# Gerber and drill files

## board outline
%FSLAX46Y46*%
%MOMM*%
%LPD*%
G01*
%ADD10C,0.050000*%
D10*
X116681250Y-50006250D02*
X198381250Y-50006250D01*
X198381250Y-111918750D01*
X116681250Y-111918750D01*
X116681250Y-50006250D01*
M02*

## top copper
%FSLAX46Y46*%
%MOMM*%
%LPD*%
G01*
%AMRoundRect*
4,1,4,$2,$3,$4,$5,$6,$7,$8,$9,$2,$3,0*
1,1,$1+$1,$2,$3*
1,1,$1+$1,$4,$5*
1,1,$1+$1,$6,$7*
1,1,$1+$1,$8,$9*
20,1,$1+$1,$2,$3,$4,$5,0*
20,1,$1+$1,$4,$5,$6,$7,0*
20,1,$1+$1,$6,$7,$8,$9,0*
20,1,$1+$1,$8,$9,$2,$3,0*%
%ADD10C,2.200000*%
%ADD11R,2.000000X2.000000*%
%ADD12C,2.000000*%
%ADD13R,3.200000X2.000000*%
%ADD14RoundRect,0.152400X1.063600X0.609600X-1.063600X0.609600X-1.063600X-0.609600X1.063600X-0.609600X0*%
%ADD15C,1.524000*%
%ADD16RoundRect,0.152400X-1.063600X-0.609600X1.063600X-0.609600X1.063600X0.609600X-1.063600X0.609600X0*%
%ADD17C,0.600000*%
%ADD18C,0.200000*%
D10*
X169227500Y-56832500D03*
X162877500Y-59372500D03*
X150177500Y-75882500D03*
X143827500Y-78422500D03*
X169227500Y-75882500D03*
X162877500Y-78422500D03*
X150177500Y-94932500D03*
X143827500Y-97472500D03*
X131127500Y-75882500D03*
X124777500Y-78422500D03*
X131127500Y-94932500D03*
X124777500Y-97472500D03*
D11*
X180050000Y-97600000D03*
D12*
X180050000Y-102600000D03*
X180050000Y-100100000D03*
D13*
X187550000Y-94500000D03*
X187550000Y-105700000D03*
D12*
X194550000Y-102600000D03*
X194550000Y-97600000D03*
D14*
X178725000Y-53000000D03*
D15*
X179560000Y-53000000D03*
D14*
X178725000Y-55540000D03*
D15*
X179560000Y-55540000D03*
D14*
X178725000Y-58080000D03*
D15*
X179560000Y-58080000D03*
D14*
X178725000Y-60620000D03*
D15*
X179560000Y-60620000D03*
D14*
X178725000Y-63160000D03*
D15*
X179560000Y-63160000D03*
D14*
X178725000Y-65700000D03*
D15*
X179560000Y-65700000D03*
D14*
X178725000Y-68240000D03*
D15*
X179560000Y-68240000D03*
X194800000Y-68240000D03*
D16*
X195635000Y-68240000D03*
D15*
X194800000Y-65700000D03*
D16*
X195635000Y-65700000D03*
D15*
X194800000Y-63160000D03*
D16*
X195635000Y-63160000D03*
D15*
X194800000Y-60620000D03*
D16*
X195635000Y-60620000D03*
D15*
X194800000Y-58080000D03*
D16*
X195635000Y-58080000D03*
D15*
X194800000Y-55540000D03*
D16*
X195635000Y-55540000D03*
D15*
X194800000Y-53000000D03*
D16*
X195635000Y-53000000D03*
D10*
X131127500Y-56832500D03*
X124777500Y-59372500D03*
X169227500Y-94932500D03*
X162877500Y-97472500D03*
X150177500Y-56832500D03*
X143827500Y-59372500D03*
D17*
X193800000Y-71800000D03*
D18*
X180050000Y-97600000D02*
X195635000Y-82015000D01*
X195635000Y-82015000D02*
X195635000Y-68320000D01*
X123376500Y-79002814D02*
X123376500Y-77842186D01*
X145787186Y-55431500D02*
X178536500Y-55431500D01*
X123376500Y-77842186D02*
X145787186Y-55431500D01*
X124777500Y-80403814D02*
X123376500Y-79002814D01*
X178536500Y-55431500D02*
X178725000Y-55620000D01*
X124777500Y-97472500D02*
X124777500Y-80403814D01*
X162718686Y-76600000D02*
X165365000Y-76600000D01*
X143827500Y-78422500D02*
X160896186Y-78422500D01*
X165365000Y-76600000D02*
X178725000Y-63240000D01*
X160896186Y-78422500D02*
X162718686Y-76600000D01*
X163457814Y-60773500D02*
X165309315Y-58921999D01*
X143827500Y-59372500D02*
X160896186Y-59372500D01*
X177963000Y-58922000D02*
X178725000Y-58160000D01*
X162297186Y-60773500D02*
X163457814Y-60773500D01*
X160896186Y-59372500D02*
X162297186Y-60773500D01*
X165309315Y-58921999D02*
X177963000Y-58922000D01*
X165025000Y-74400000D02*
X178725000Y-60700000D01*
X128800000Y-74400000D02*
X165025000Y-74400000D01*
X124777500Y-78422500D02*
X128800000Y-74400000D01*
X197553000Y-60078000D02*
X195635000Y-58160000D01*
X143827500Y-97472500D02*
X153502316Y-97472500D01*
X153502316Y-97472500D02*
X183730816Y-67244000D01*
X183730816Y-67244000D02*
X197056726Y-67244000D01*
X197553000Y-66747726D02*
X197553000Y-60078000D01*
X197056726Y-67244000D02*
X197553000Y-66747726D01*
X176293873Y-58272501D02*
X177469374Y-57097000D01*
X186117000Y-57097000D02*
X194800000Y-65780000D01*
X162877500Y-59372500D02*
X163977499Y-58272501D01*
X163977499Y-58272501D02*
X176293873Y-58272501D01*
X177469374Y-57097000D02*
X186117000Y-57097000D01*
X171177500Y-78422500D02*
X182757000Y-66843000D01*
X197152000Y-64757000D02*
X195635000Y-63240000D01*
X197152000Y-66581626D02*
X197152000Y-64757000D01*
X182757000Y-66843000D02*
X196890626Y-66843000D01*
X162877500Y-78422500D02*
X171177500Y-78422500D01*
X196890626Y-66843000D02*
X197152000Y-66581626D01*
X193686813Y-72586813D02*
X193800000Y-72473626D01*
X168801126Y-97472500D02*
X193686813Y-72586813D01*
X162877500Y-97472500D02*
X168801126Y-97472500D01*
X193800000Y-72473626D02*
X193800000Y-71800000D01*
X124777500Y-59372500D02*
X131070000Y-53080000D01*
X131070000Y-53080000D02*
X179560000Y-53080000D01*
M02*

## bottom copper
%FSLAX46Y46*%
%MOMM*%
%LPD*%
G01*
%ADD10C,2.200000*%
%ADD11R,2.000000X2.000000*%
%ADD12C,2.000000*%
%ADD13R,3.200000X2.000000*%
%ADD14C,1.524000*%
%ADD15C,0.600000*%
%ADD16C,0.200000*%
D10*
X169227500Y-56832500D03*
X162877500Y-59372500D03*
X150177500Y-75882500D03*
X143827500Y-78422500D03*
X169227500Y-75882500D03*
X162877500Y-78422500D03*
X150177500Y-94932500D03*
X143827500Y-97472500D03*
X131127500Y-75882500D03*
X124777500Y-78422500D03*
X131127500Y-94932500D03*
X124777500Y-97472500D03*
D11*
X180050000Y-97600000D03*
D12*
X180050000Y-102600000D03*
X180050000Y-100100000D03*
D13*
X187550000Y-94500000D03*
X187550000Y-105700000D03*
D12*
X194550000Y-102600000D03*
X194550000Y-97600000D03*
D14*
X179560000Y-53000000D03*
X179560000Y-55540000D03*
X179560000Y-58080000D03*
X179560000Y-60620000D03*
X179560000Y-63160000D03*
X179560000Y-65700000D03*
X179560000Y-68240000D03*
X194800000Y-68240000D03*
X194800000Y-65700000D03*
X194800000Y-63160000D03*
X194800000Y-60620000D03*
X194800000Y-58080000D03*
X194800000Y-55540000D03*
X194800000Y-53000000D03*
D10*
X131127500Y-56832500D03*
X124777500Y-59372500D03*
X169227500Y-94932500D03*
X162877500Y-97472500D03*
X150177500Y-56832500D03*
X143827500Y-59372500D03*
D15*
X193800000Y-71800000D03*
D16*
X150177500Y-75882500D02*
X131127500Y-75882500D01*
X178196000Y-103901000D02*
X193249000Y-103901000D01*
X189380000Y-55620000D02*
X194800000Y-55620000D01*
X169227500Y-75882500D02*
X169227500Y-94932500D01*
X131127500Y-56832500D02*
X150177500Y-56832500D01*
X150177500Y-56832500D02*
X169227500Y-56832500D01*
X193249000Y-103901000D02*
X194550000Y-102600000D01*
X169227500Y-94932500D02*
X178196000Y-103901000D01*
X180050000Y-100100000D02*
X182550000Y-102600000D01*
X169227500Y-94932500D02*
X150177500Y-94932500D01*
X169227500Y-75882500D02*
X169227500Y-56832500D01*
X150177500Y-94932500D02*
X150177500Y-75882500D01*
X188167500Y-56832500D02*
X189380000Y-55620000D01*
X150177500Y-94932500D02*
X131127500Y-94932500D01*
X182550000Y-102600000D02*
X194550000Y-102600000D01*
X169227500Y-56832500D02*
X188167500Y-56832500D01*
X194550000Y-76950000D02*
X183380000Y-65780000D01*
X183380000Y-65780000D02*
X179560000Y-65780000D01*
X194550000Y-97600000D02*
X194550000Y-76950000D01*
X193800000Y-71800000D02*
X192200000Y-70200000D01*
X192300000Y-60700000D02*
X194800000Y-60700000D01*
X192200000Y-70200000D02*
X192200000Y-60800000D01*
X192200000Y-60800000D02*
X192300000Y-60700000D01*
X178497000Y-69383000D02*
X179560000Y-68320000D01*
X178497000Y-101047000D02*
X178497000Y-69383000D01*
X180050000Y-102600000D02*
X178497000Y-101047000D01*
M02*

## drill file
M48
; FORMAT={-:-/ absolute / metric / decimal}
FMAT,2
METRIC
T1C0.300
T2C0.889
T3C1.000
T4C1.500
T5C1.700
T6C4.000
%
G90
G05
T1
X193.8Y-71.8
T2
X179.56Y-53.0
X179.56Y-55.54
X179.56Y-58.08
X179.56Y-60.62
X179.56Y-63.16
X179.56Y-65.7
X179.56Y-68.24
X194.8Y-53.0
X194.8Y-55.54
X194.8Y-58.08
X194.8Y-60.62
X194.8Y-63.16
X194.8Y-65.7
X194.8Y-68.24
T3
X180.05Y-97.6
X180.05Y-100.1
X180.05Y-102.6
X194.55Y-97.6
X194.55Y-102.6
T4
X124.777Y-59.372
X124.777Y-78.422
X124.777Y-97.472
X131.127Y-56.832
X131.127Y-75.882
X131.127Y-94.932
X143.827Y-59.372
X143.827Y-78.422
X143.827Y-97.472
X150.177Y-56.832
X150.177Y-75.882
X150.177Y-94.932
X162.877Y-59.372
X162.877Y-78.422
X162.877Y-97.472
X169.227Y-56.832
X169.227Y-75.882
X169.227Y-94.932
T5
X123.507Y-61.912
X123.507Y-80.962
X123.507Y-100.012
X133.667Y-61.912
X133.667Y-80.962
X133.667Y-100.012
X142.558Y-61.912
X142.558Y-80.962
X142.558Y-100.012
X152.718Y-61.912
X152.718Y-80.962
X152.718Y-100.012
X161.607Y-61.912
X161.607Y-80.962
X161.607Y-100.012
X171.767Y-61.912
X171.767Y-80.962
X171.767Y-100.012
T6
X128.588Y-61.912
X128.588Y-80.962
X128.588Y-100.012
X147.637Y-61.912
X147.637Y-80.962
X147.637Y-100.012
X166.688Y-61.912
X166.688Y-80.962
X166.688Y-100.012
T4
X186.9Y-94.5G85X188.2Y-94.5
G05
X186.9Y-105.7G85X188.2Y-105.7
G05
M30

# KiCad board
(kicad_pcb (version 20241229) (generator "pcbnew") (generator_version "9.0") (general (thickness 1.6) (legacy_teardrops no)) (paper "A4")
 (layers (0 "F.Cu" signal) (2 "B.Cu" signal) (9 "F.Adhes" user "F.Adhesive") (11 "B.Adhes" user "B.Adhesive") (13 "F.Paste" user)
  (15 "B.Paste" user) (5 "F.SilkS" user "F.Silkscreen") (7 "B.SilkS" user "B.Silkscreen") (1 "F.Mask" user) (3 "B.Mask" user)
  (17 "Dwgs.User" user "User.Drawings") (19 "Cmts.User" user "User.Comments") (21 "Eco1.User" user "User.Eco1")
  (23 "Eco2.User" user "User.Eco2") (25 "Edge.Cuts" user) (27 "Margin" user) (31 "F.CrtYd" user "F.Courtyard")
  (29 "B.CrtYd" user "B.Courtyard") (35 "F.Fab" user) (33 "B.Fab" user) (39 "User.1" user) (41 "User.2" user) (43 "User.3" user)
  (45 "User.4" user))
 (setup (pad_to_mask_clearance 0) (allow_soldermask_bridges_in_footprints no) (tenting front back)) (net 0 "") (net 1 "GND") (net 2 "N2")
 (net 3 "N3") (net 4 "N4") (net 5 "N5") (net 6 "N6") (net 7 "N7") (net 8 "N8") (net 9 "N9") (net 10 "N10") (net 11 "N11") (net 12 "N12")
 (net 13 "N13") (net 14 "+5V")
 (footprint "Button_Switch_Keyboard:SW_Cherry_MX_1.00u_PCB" (layer "F.Cu") (at 169.2275 56.8325)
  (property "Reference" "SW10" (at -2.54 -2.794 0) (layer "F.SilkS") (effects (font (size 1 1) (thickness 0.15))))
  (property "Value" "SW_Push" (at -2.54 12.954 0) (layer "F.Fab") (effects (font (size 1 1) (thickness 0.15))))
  (pad "" np_thru_hole circle (at -7.62 5.08) (size 1.7 1.7) (drill 1.7) (layers "*.Cu" "*.Mask"))
  (pad "" np_thru_hole circle (at -2.54 5.08) (size 4 4) (drill 4) (layers "*.Cu" "*.Mask"))
  (pad "" np_thru_hole circle (at 2.54 5.08) (size 1.7 1.7) (drill 1.7) (layers "*.Cu" "*.Mask"))
  (pad "1" thru_hole circle (at 0 0) (size 2.2 2.2) (drill 1.5) (layers "*.Cu" "*.Mask") (remove_unused_layers no) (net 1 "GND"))
  (pad "2" thru_hole circle (at -6.35 2.54) (size 2.2 2.2) (drill 1.5) (layers "*.Cu" "*.Mask") (remove_unused_layers no) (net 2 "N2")))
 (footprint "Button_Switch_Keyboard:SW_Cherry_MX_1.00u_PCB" (layer "F.Cu") (at 150.1775 75.8825)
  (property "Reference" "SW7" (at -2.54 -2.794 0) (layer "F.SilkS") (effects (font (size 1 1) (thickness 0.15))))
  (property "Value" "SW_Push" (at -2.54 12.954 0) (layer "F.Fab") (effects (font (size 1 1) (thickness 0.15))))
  (pad "" np_thru_hole circle (at -7.62 5.08) (size 1.7 1.7) (drill 1.7) (layers "*.Cu" "*.Mask"))
  (pad "" np_thru_hole circle (at -2.54 5.08) (size 4 4) (drill 4) (layers "*.Cu" "*.Mask"))
  (pad "" np_thru_hole circle (at 2.54 5.08) (size 1.7 1.7) (drill 1.7) (layers "*.Cu" "*.Mask"))
  (pad "1" thru_hole circle (at 0 0) (size 2.2 2.2) (drill 1.5) (layers "*.Cu" "*.Mask") (remove_unused_layers no) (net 1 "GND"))
  (pad "2" thru_hole circle (at -6.35 2.54) (size 2.2 2.2) (drill 1.5) (layers "*.Cu" "*.Mask") (remove_unused_layers no) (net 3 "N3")))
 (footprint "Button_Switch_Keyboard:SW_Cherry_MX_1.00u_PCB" (layer "F.Cu") (at 169.2275 75.8825)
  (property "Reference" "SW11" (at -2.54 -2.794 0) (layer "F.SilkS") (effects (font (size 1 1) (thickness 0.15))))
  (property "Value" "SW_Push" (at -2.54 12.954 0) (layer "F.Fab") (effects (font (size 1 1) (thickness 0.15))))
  (pad "" np_thru_hole circle (at -7.62 5.08) (size 1.7 1.7) (drill 1.7) (layers "*.Cu" "*.Mask"))
  (pad "" np_thru_hole circle (at -2.54 5.08) (size 4 4) (drill 4) (layers "*.Cu" "*.Mask"))
  (pad "" np_thru_hole circle (at 2.54 5.08) (size 1.7 1.7) (drill 1.7) (layers "*.Cu" "*.Mask"))
  (pad "1" thru_hole circle (at 0 0) (size 2.2 2.2) (drill 1.5) (layers "*.Cu" "*.Mask") (remove_unused_layers no) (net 1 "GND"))
  (pad "2" thru_hole circle (at -6.35 2.54) (size 2.2 2.2) (drill 1.5) (layers "*.Cu" "*.Mask") (remove_unused_layers no) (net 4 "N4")))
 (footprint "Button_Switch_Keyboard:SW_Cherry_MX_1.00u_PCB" (layer "F.Cu") (at 150.1775 94.9325)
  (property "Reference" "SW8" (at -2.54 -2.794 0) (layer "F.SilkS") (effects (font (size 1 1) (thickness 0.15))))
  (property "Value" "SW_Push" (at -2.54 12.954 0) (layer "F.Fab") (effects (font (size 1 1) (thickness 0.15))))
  (pad "" np_thru_hole circle (at -7.62 5.08) (size 1.7 1.7) (drill 1.7) (layers "*.Cu" "*.Mask"))
  (pad "" np_thru_hole circle (at -2.54 5.08) (size 4 4) (drill 4) (layers "*.Cu" "*.Mask"))
  (pad "" np_thru_hole circle (at 2.54 5.08) (size 1.7 1.7) (drill 1.7) (layers "*.Cu" "*.Mask"))
  (pad "1" thru_hole circle (at 0 0) (size 2.2 2.2) (drill 1.5) (layers "*.Cu" "*.Mask") (remove_unused_layers no) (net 1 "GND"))
  (pad "2" thru_hole circle (at -6.35 2.54) (size 2.2 2.2) (drill 1.5) (layers "*.Cu" "*.Mask") (remove_unused_layers no) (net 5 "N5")))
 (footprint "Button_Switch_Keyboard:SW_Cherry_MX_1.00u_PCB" (layer "F.Cu") (at 131.1275 75.8825)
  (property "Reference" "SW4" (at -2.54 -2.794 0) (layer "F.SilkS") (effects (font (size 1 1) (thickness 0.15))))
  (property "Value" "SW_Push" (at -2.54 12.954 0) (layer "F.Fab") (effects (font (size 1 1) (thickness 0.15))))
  (pad "" np_thru_hole circle (at -7.62 5.08) (size 1.7 1.7) (drill 1.7) (layers "*.Cu" "*.Mask"))
  (pad "" np_thru_hole circle (at -2.54 5.08) (size 4 4) (drill 4) (layers "*.Cu" "*.Mask"))
  (pad "" np_thru_hole circle (at 2.54 5.08) (size 1.7 1.7) (drill 1.7) (layers "*.Cu" "*.Mask"))
  (pad "1" thru_hole circle (at 0 0) (size 2.2 2.2) (drill 1.5) (layers "*.Cu" "*.Mask") (remove_unused_layers no) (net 1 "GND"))
  (pad "2" thru_hole circle (at -6.35 2.54) (size 2.2 2.2) (drill 1.5) (layers "*.Cu" "*.Mask") (remove_unused_layers no) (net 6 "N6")))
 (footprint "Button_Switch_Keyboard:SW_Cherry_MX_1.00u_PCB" (layer "F.Cu") (at 131.1275 94.9325)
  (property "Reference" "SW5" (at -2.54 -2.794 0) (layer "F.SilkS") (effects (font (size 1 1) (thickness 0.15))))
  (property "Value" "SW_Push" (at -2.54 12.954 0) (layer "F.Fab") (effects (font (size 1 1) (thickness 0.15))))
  (pad "" np_thru_hole circle (at -7.62 5.08) (size 1.7 1.7) (drill 1.7) (layers "*.Cu" "*.Mask"))
  (pad "" np_thru_hole circle (at -2.54 5.08) (size 4 4) (drill 4) (layers "*.Cu" "*.Mask"))
  (pad "" np_thru_hole circle (at 2.54 5.08) (size 1.7 1.7) (drill 1.7) (layers "*.Cu" "*.Mask"))
  (pad "1" thru_hole circle (at 0 0) (size 2.2 2.2) (drill 1.5) (layers "*.Cu" "*.Mask") (remove_unused_layers no) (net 1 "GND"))
  (pad "2" thru_hole circle (at -6.35 2.54) (size 2.2 2.2) (drill 1.5) (layers "*.Cu" "*.Mask") (remove_unused_layers no) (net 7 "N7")))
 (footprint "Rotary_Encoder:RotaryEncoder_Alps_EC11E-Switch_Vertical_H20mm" (layer "F.Cu") (at 180.05 97.6)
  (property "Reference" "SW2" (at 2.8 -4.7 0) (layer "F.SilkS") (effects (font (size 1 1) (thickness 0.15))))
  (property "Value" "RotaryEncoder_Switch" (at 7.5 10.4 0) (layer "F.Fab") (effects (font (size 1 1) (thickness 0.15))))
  (pad "A" thru_hole rect (at 0 0) (size 2 2) (drill 1) (layers "*.Cu" "*.Mask") (remove_unused_layers no) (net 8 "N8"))
  (pad "B" thru_hole circle (at 0 5) (size 2 2) (drill 1) (layers "*.Cu" "*.Mask") (remove_unused_layers no) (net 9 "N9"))
  (pad "C" thru_hole circle (at 0 2.5) (size 2 2) (drill 1) (layers "*.Cu" "*.Mask") (remove_unused_layers no) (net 1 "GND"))
  (pad "MP" thru_hole rect (at 7.5 -3.1) (size 3.2 2) (drill oval 2.8 1.5) (layers "*.Cu" "*.Mask") (remove_unused_layers no))
  (pad "MP" thru_hole rect (at 7.5 8.1) (size 3.2 2) (drill oval 2.8 1.5) (layers "*.Cu" "*.Mask") (remove_unused_layers no))
  (pad "S1" thru_hole circle (at 14.5 5) (size 2 2) (drill 1) (layers "*.Cu" "*.Mask") (remove_unused_layers no) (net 1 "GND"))
  (pad "S2" thru_hole circle (at 14.5 0) (size 2 2) (drill 1) (layers "*.Cu" "*.Mask") (remove_unused_layers no) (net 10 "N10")))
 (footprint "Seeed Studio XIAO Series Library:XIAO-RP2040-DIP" (layer "F.Cu") (at 187.18 60.62)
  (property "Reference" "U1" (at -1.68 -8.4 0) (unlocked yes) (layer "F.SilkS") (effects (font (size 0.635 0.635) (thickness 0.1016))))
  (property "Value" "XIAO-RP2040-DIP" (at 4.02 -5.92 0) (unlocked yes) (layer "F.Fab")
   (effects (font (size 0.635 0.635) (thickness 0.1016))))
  (pad "1" smd roundrect (at -8.455 -7.62 180) (size 2.432 1.524) (layers "F.Cu" "F.Mask") (roundrect_rratio 0.1) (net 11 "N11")
   (thermal_bridge_angle 45))
  (pad "1" thru_hole circle (at -7.62 -7.62 180) (size 1.524 1.524) (drill 0.889) (layers "*.Cu" "*.Mask") (remove_unused_layers no)
   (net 11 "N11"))
  (pad "2" smd roundrect (at -8.455 -5.08 180) (size 2.432 1.524) (layers "F.Cu" "F.Mask") (roundrect_rratio 0.1) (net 7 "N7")
   (thermal_bridge_angle 45))
  (pad "2" thru_hole circle (at -7.62 -5.08 180) (size 1.524 1.524) (drill 0.889) (layers "*.Cu" "*.Mask") (remove_unused_layers no)
   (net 7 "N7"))
  (pad "3" smd roundrect (at -8.455 -2.54 180) (size 2.432 1.524) (layers "F.Cu" "F.Mask") (roundrect_rratio 0.1) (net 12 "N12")
   (thermal_bridge_angle 45))
  (pad "3" thru_hole circle (at -7.62 -2.54 180) (size 1.524 1.524) (drill 0.889) (layers "*.Cu" "*.Mask") (remove_unused_layers no)
   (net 12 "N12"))
  (pad "4" smd roundrect (at -8.455 0 180) (size 2.432 1.524) (layers "F.Cu" "F.Mask") (roundrect_rratio 0.1) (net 6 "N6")
   (thermal_bridge_angle 45))
  (pad "4" thru_hole circle (at -7.62 0 180) (size 1.524 1.524) (drill 0.889) (layers "*.Cu" "*.Mask") (remove_unused_layers no)
   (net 6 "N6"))
  (pad "5" smd roundrect (at -8.455 2.54 180) (size 2.432 1.524) (layers "F.Cu" "F.Mask") (roundrect_rratio 0.1) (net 3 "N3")
   (thermal_bridge_angle 45))
  (pad "5" thru_hole circle (at -7.62 2.54 180) (size 1.524 1.524) (drill 0.889) (layers "*.Cu" "*.Mask") (remove_unused_layers no)
   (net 3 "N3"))
  (pad "6" smd roundrect (at -8.455 5.08 180) (size 2.432 1.524) (layers "F.Cu" "F.Mask") (roundrect_rratio 0.1) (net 10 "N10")
   (thermal_bridge_angle 45))
  (pad "6" thru_hole circle (at -7.62 5.08 180) (size 1.524 1.524) (drill 0.889) (layers "*.Cu" "*.Mask") (remove_unused_layers no)
   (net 10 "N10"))
  (pad "7" smd roundrect (at -8.455 7.62 180) (size 2.432 1.524) (layers "F.Cu" "F.Mask") (roundrect_rratio 0.1) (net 9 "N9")
   (thermal_bridge_angle 45))
  (pad "7" thru_hole circle (at -7.62 7.62 180) (size 1.524 1.524) (drill 0.889) (layers "*.Cu" "*.Mask") (remove_unused_layers no)
   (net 9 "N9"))
  (pad "8" thru_hole circle (at 7.62 7.62) (size 1.524 1.524) (drill 0.889) (layers "*.Cu" "*.Mask") (remove_unused_layers no) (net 8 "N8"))
  (pad "8" smd roundrect (at 8.455 7.62) (size 2.432 1.524) (layers "F.Cu" "F.Mask") (roundrect_rratio 0.1) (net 8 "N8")
   (thermal_bridge_angle 45))
  (pad "9" thru_hole circle (at 7.62 5.08) (size 1.524 1.524) (drill 0.889) (layers "*.Cu" "*.Mask") (remove_unused_layers no) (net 2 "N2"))
  (pad "9" smd roundrect (at 8.455 5.08) (size 2.432 1.524) (layers "F.Cu" "F.Mask") (roundrect_rratio 0.1) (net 2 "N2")
   (thermal_bridge_angle 45))
  (pad "10" thru_hole circle (at 7.62 2.54) (size 1.524 1.524) (drill 0.889) (layers "*.Cu" "*.Mask") (remove_unused_layers no) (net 4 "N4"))
  (pad "10" smd roundrect (at 8.455 2.54) (size 2.432 1.524) (layers "F.Cu" "F.Mask") (roundrect_rratio 0.1) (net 4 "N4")
   (thermal_bridge_angle 45))
  (pad "11" thru_hole circle (at 7.62 0) (size 1.524 1.524) (drill 0.889) (layers "*.Cu" "*.Mask") (remove_unused_layers no) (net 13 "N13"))
  (pad "11" smd roundrect (at 8.455 0) (size 2.432 1.524) (layers "F.Cu" "F.Mask") (roundrect_rratio 0.1) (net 13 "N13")
   (thermal_bridge_angle 45))
  (pad "12" thru_hole circle (at 7.62 -2.54) (size 1.524 1.524) (drill 0.889) (layers "*.Cu" "*.Mask") (remove_unused_layers no)
   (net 5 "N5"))
  (pad "12" smd roundrect (at 8.455 -2.54) (size 2.432 1.524) (layers "F.Cu" "F.Mask") (roundrect_rratio 0.1) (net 5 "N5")
   (thermal_bridge_angle 45))
  (pad "13" thru_hole circle (at 7.62 -5.08) (size 1.524 1.524) (drill 0.889) (layers "*.Cu" "*.Mask") (remove_unused_layers no)
   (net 1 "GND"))
  (pad "13" smd roundrect (at 8.455 -5.08) (size 2.432 1.524) (layers "F.Cu" "F.Mask") (roundrect_rratio 0.1) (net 1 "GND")
   (thermal_bridge_angle 45))
  (pad "14" thru_hole circle (at 7.62 -7.62) (size 1.524 1.524) (drill 0.889) (layers "*.Cu" "*.Mask") (remove_unused_layers no)
   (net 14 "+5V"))
  (pad "14" smd roundrect (at 8.455 -7.62) (size 2.432 1.524) (layers "F.Cu" "F.Mask") (roundrect_rratio 0.1) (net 14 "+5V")
   (thermal_bridge_angle 45)))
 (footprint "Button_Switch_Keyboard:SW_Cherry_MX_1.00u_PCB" (layer "F.Cu") (at 131.1275 56.8325)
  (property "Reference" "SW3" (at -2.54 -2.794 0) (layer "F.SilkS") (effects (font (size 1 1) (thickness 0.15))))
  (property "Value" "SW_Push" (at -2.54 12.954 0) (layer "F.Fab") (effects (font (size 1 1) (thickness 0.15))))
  (pad "" np_thru_hole circle (at -7.62 5.08) (size 1.7 1.7) (drill 1.7) (layers "*.Cu" "*.Mask"))
  (pad "" np_thru_hole circle (at -2.54 5.08) (size 4 4) (drill 4) (layers "*.Cu" "*.Mask"))
  (pad "" np_thru_hole circle (at 2.54 5.08) (size 1.7 1.7) (drill 1.7) (layers "*.Cu" "*.Mask"))
  (pad "1" thru_hole circle (at 0 0) (size 2.2 2.2) (drill 1.5) (layers "*.Cu" "*.Mask") (remove_unused_layers no) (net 1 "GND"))
  (pad "2" thru_hole circle (at -6.35 2.54) (size 2.2 2.2) (drill 1.5) (layers "*.Cu" "*.Mask") (remove_unused_layers no) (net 11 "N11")))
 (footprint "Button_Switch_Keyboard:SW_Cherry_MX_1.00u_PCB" (layer "F.Cu") (at 169.2275 94.9325)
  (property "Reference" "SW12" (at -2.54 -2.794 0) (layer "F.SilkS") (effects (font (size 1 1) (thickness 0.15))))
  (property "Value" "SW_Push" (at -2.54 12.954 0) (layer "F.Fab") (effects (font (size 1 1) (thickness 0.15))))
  (pad "" np_thru_hole circle (at -7.62 5.08) (size 1.7 1.7) (drill 1.7) (layers "*.Cu" "*.Mask"))
  (pad "" np_thru_hole circle (at -2.54 5.08) (size 4 4) (drill 4) (layers "*.Cu" "*.Mask"))
  (pad "" np_thru_hole circle (at 2.54 5.08) (size 1.7 1.7) (drill 1.7) (layers "*.Cu" "*.Mask"))
  (pad "1" thru_hole circle (at 0 0) (size 2.2 2.2) (drill 1.5) (layers "*.Cu" "*.Mask") (remove_unused_layers no) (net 1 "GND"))
  (pad "2" thru_hole circle (at -6.35 2.54) (size 2.2 2.2) (drill 1.5) (layers "*.Cu" "*.Mask") (remove_unused_layers no) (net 13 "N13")))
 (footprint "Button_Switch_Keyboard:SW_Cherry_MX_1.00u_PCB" (layer "F.Cu") (at 150.1775 56.8325)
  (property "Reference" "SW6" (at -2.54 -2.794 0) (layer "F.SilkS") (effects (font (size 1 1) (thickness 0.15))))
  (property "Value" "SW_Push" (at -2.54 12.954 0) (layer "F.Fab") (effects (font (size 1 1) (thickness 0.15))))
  (pad "" np_thru_hole circle (at -7.62 5.08) (size 1.7 1.7) (drill 1.7) (layers "*.Cu" "*.Mask"))
  (pad "" np_thru_hole circle (at -2.54 5.08) (size 4 4) (drill 4) (layers "*.Cu" "*.Mask"))
  (pad "" np_thru_hole circle (at 2.54 5.08) (size 1.7 1.7) (drill 1.7) (layers "*.Cu" "*.Mask"))
  (pad "1" thru_hole circle (at 0 0) (size 2.2 2.2) (drill 1.5) (layers "*.Cu" "*.Mask") (remove_unused_layers no) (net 1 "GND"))
  (pad "2" thru_hole circle (at -6.35 2.54) (size 2.2 2.2) (drill 1.5) (layers "*.Cu" "*.Mask") (remove_unused_layers no) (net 12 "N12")))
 (gr_rect (start 116.68125 50.00625) (end 198.38125 111.91875) (stroke (width 0.05) (type default)) (fill no) (layer "Edge.Cuts"))
 (segment (start 150.1775 75.8825) (end 131.1275 75.8825) (width 0.2) (layer "B.Cu") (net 1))
 (segment (start 178.196 103.901) (end 193.249 103.901) (width 0.2) (layer "B.Cu") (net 1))
 (segment (start 189.38 55.62) (end 194.8 55.62) (width 0.2) (layer "B.Cu") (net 1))
 (segment (start 169.2275 75.8825) (end 169.2275 94.9325) (width 0.2) (layer "B.Cu") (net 1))
 (segment (start 131.1275 56.8325) (end 150.1775 56.8325) (width 0.2) (layer "B.Cu") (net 1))
 (segment (start 150.1775 56.8325) (end 169.2275 56.8325) (width 0.2) (layer "B.Cu") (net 1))
 (segment (start 193.249 103.901) (end 194.55 102.6) (width 0.2) (layer "B.Cu") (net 1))
 (segment (start 169.2275 94.9325) (end 178.196 103.901) (width 0.2) (layer "B.Cu") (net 1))
 (segment (start 180.05 100.1) (end 182.55 102.6) (width 0.2) (layer "B.Cu") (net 1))
 (segment (start 169.2275 94.9325) (end 150.1775 94.9325) (width 0.2) (layer "B.Cu") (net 1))
 (segment (start 169.2275 75.8825) (end 169.2275 56.8325) (width 0.2) (layer "B.Cu") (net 1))
 (segment (start 150.1775 94.9325) (end 150.1775 75.8825) (width 0.2) (layer "B.Cu") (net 1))
 (segment (start 188.1675 56.8325) (end 189.38 55.62) (width 0.2) (layer "B.Cu") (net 1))
 (segment (start 150.1775 94.9325) (end 131.1275 94.9325) (width 0.2) (layer "B.Cu") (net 1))
 (segment (start 182.55 102.6) (end 194.55 102.6) (width 0.2) (layer "B.Cu") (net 1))
 (segment (start 169.2275 56.8325) (end 188.1675 56.8325) (width 0.2) (layer "B.Cu") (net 1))
 (segment (start 180.05 97.6) (end 195.635 82.015) (width 0.2) (layer "F.Cu") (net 8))
 (segment (start 195.635 82.015) (end 195.635 68.32) (width 0.2) (layer "F.Cu") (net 8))
 (segment (start 123.3765 79.002814) (end 123.3765 77.842186) (width 0.2) (layer "F.Cu") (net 7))
 (segment (start 145.787186 55.4315) (end 178.5365 55.4315) (width 0.2) (layer "F.Cu") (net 7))
 (segment (start 123.3765 77.842186) (end 145.787186 55.4315) (width 0.2) (layer "F.Cu") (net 7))
 (segment (start 124.7775 80.403814) (end 123.3765 79.002814) (width 0.2) (layer "F.Cu") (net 7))
 (segment (start 178.5365 55.4315) (end 178.725 55.62) (width 0.2) (layer "F.Cu") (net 7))
 (segment (start 124.7775 97.4725) (end 124.7775 80.403814) (width 0.2) (layer "F.Cu") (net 7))
 (segment (start 162.718686 76.6) (end 165.365 76.6) (width 0.2) (layer "F.Cu") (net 3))
 (segment (start 143.8275 78.4225) (end 160.896186 78.4225) (width 0.2) (layer "F.Cu") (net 3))
 (segment (start 165.365 76.6) (end 178.725 63.24) (width 0.2) (layer "F.Cu") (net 3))
 (segment (start 160.896186 78.4225) (end 162.718686 76.6) (width 0.2) (layer "F.Cu") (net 3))
 (segment (start 163.457814 60.7735) (end 165.309315 58.921999) (width 0.2) (layer "F.Cu") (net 12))
 (segment (start 143.8275 59.3725) (end 160.896186 59.3725) (width 0.2) (layer "F.Cu") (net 12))
 (segment (start 177.963 58.922) (end 178.725 58.16) (width 0.2) (layer "F.Cu") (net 12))
 (segment (start 162.297186 60.7735) (end 163.457814 60.7735) (width 0.2) (layer "F.Cu") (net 12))
 (segment (start 160.896186 59.3725) (end 162.297186 60.7735) (width 0.2) (layer "F.Cu") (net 12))
 (segment (start 165.309315 58.921999) (end 177.963 58.922) (width 0.2) (layer "F.Cu") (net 12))
 (segment (start 165.025 74.4) (end 178.725 60.7) (width 0.2) (layer "F.Cu") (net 6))
 (segment (start 128.8 74.4) (end 165.025 74.4) (width 0.2) (layer "F.Cu") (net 6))
 (segment (start 124.7775 78.4225) (end 128.8 74.4) (width 0.2) (layer "F.Cu") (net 6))
 (segment (start 194.55 76.95) (end 183.38 65.78) (width 0.2) (layer "B.Cu") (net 10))
 (segment (start 183.38 65.78) (end 179.56 65.78) (width 0.2) (layer "B.Cu") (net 10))
 (segment (start 194.55 97.6) (end 194.55 76.95) (width 0.2) (layer "B.Cu") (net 10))
 (segment (start 197.553 60.078) (end 195.635 58.16) (width 0.2) (layer "F.Cu") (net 5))
 (segment (start 143.8275 97.4725) (end 153.502316 97.4725) (width 0.2) (layer "F.Cu") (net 5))
 (segment (start 153.502316 97.4725) (end 183.730816 67.244) (width 0.2) (layer "F.Cu") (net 5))
 (segment (start 183.730816 67.244) (end 197.056726 67.244) (width 0.2) (layer "F.Cu") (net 5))
 (segment (start 197.553 66.747726) (end 197.553 60.078) (width 0.2) (layer "F.Cu") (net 5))
 (segment (start 197.056726 67.244) (end 197.553 66.747726) (width 0.2) (layer "F.Cu") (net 5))
 (segment (start 176.293873 58.272501) (end 177.469374 57.097) (width 0.2) (layer "F.Cu") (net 2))
 (segment (start 186.117 57.097) (end 194.8 65.78) (width 0.2) (layer "F.Cu") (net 2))
 (segment (start 162.8775 59.3725) (end 163.977499 58.272501) (width 0.2) (layer "F.Cu") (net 2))
 (segment (start 163.977499 58.272501) (end 176.293873 58.272501) (width 0.2) (layer "F.Cu") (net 2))
 (segment (start 177.469374 57.097) (end 186.117 57.097) (width 0.2) (layer "F.Cu") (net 2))
 (segment (start 171.1775 78.4225) (end 182.757 66.843) (width 0.2) (layer "F.Cu") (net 4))
 (segment (start 197.152 64.757) (end 195.635 63.24) (width 0.2) (layer "F.Cu") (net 4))
 (segment (start 197.152 66.581626) (end 197.152 64.757) (width 0.2) (layer "F.Cu") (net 4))
 (segment (start 182.757 66.843) (end 196.890626 66.843) (width 0.2) (layer "F.Cu") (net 4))
 (segment (start 162.8775 78.4225) (end 171.1775 78.4225) (width 0.2) (layer "F.Cu") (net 4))
 (segment (start 196.890626 66.843) (end 197.152 66.581626) (width 0.2) (layer "F.Cu") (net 4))
 (segment (start 193.686813 72.586813) (end 193.8 72.473626) (width 0.2) (layer "F.Cu") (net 13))
 (segment (start 168.801126 97.4725) (end 193.686813 72.586813) (width 0.2) (layer "F.Cu") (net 13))
 (segment (start 162.8775 97.4725) (end 168.801126 97.4725) (width 0.2) (layer "F.Cu") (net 13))
 (segment (start 193.8 72.473626) (end 193.8 71.8) (width 0.2) (layer "F.Cu") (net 13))
 (via (at 193.8 71.8) (size 0.6) (drill 0.3) (layers "F.Cu" "B.Cu") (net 13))
 (segment (start 193.8 71.8) (end 192.2 70.2) (width 0.2) (layer "B.Cu") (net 13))
 (segment (start 192.3 60.7) (end 194.8 60.7) (width 0.2) (layer "B.Cu") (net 13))
 (segment (start 192.2 70.2) (end 192.2 60.8) (width 0.2) (layer "B.Cu") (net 13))
 (segment (start 192.2 60.8) (end 192.3 60.7) (width 0.2) (layer "B.Cu") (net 13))
 (segment (start 178.497 69.383) (end 179.56 68.32) (width 0.2) (layer "B.Cu") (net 9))
 (segment (start 178.497 101.047) (end 178.497 69.383) (width 0.2) (layer "B.Cu") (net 9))
 (segment (start 180.05 102.6) (end 178.497 101.047) (width 0.2) (layer "B.Cu") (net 9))
 (segment (start 124.7775 59.3725) (end 131.07 53.08) (width 0.2) (layer "F.Cu") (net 11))
 (segment (start 131.07 53.08) (end 179.56 53.08) (width 0.2) (layer "F.Cu") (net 11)))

